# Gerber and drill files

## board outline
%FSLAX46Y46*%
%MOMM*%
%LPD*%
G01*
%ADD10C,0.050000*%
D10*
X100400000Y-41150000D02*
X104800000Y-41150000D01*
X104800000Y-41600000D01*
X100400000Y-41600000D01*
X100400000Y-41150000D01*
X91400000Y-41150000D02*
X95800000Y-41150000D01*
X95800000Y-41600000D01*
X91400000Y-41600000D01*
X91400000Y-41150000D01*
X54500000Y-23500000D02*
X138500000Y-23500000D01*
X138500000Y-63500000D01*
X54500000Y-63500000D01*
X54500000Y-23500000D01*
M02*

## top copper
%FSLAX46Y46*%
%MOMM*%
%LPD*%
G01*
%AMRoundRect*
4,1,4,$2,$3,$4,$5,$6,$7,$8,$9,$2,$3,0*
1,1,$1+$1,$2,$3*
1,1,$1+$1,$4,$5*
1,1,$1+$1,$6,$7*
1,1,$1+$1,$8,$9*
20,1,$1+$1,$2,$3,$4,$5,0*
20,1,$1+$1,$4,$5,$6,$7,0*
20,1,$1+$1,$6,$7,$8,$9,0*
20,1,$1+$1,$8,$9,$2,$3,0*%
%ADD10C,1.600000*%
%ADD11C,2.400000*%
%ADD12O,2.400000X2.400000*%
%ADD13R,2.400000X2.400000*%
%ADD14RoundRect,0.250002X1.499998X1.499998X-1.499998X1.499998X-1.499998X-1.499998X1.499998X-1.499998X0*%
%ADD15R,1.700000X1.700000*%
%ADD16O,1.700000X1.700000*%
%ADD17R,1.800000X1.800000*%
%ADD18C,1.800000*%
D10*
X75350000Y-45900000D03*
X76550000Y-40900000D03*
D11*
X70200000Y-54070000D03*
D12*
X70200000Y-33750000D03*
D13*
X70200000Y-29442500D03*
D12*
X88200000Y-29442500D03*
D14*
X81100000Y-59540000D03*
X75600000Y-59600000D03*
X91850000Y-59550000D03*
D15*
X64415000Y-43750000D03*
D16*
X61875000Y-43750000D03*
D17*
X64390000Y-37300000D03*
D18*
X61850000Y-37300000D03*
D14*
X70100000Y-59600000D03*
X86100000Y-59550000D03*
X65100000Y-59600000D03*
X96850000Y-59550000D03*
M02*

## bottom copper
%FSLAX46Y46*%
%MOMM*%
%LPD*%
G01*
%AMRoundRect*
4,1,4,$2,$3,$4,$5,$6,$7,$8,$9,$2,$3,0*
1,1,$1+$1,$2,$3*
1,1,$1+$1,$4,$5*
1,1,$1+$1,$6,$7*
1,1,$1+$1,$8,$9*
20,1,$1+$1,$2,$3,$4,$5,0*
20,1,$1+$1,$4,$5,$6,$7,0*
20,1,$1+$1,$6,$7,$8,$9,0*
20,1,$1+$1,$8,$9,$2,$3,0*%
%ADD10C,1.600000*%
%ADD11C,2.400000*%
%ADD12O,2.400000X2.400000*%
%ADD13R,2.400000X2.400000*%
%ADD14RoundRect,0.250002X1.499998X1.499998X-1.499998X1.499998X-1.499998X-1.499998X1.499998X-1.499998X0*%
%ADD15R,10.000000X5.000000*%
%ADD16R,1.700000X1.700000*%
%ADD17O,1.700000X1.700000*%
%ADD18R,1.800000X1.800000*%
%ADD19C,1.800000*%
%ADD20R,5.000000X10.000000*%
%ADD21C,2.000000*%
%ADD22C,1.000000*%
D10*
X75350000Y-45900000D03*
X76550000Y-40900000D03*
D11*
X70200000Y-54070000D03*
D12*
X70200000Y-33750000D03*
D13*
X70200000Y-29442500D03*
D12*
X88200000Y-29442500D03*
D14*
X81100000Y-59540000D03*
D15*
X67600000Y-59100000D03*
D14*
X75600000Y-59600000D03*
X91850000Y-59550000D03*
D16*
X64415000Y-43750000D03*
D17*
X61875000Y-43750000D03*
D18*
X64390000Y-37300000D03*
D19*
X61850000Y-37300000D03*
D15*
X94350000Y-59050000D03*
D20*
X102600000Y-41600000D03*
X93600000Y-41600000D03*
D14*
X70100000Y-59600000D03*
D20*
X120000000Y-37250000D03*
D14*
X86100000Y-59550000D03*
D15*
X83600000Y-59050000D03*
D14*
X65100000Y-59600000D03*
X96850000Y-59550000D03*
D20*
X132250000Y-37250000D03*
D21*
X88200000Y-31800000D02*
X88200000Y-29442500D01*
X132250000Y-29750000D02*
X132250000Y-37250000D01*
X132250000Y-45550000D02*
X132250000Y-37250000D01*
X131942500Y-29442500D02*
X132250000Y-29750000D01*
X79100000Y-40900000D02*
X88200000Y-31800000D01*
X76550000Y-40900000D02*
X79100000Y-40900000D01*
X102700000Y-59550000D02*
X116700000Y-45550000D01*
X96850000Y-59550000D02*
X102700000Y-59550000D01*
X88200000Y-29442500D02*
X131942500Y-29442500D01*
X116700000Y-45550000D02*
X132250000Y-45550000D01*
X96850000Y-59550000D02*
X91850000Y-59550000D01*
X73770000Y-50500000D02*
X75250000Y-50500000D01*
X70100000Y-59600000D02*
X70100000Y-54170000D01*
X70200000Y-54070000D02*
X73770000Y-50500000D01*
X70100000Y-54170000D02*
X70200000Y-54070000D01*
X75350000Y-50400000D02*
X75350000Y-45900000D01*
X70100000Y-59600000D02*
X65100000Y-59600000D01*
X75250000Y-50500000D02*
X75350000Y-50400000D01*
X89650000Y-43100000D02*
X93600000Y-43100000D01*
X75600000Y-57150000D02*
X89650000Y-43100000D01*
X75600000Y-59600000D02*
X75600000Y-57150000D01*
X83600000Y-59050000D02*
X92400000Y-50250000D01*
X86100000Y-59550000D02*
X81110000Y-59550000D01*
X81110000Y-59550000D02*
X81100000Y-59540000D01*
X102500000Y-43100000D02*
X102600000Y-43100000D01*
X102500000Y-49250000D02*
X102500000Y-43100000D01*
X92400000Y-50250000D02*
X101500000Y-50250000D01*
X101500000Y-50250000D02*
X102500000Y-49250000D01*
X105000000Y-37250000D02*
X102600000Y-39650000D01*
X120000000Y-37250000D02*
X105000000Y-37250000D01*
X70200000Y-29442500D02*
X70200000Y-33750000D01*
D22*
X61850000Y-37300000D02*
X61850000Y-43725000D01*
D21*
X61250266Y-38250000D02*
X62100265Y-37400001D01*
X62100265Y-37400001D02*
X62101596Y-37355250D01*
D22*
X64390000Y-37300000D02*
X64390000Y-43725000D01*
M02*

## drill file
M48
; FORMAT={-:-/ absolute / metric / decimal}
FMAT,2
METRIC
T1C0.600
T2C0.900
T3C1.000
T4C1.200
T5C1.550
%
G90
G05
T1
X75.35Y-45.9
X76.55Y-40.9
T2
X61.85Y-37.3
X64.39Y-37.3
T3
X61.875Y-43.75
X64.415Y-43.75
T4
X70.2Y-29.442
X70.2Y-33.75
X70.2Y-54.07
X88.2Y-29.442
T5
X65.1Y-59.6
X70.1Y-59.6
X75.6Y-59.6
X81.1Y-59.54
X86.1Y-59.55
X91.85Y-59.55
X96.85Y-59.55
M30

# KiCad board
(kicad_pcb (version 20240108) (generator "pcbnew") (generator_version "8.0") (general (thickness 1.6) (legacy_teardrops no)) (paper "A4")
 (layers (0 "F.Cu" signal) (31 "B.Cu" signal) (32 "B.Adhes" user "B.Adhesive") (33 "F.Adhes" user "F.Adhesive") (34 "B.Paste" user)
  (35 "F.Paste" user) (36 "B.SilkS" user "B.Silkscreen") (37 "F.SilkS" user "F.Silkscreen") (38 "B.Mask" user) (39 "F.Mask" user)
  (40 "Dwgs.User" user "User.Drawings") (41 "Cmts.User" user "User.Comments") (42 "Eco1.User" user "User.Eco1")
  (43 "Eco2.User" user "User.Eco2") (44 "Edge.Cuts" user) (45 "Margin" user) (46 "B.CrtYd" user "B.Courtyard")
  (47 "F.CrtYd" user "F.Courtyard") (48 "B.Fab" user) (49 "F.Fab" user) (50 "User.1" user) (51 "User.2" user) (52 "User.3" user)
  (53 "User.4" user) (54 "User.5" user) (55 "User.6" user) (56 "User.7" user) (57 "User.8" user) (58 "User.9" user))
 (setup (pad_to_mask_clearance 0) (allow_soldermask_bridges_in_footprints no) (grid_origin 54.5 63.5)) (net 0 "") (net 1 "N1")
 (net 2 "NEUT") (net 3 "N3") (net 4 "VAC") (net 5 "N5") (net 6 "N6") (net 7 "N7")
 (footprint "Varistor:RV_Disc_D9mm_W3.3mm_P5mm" (layer "F.Cu") (at 75.35 45.9 90)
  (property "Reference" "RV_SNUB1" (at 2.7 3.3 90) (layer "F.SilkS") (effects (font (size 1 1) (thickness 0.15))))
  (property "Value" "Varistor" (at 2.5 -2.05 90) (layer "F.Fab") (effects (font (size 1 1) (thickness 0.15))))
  (pad "1" thru_hole circle (at 0 0 90) (size 1.6 1.6) (drill 0.6) (layers "*.Cu" "*.Mask") (remove_unused_layers no) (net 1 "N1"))
  (pad "2" thru_hole circle (at 5 1.2 90) (size 1.6 1.6) (drill 0.6) (layers "*.Cu" "*.Mask") (remove_unused_layers no) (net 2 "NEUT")))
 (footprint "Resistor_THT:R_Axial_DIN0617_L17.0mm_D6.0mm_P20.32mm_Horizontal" (layer "F.Cu") (at 70.2 54.07 90)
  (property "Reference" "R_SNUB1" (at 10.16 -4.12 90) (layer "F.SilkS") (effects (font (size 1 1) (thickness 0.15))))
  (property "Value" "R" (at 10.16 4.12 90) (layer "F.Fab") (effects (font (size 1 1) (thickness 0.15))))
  (pad "1" thru_hole circle (at 0 0 90) (size 2.4 2.4) (drill 1.2) (layers "*.Cu" "*.Mask") (remove_unused_layers no) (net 1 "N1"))
  (pad "2" thru_hole oval (at 20.32 0 90) (size 2.4 2.4) (drill 1.2) (layers "*.Cu" "*.Mask") (remove_unused_layers no) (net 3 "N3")))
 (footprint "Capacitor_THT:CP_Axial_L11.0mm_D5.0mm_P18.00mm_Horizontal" (layer "F.Cu") (at 70.2 29.4425)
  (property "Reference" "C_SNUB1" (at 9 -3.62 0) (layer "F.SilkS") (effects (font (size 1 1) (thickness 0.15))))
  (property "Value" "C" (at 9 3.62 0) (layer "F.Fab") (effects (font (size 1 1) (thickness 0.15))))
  (pad "1" thru_hole rect (at 0 0) (size 2.4 2.4) (drill 1.2) (layers "*.Cu" "*.Mask") (remove_unused_layers no) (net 3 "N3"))
  (pad "2" thru_hole oval (at 18 0) (size 2.4 2.4) (drill 1.2) (layers "*.Cu" "*.Mask") (remove_unused_layers no) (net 2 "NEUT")))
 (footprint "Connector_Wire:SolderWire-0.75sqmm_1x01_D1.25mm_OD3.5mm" (layer "B.Cu") (at 81.1 59.54 180)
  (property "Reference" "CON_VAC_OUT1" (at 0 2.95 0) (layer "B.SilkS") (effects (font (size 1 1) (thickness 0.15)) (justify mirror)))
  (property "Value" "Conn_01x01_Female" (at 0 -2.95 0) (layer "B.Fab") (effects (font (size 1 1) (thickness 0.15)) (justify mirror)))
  (pad "1" thru_hole roundrect (at 0 0 180) (size 3.5 3.5) (drill 1.55) (layers "*.Cu" "*.Mask") (remove_unused_layers no)
   (roundrect_rratio 0.071429) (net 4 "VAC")))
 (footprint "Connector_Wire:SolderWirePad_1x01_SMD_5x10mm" (layer "B.Cu") (at 67.6 59.1 90)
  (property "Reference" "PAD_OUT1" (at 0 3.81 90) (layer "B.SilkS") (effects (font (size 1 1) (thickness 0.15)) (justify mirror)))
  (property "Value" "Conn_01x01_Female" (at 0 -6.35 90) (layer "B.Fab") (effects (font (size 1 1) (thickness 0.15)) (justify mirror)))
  (pad "1" smd rect (at 0 0 90) (size 5 10) (layers "B.Cu" "B.Paste" "B.Mask") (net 1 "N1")))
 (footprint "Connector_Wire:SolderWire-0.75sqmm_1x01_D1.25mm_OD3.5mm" (layer "B.Cu") (at 75.6 59.6 180)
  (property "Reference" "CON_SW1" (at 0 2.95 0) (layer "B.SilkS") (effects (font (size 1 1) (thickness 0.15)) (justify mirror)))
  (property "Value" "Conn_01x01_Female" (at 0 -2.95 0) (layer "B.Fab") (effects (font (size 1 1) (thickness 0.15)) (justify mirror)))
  (pad "1" thru_hole roundrect (at 0 0 180) (size 3.5 3.5) (drill 1.55) (layers "*.Cu" "*.Mask") (remove_unused_layers no)
   (roundrect_rratio 0.071429) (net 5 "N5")))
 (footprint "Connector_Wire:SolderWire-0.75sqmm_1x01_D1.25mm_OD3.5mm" (layer "B.Cu") (at 91.85 59.55 180)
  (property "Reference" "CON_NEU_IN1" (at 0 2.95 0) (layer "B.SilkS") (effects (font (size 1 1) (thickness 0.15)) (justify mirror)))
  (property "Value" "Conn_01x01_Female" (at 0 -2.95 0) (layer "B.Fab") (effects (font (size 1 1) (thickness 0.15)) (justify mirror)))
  (pad "1" thru_hole roundrect (at 0 0 180) (size 3.5 3.5) (drill 1.55) (layers "*.Cu" "*.Mask") (remove_unused_layers no)
   (roundrect_rratio 0.071429) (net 2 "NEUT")))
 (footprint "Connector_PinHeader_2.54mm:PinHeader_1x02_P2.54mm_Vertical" (layer "B.Cu") (at 64.415 43.75 90)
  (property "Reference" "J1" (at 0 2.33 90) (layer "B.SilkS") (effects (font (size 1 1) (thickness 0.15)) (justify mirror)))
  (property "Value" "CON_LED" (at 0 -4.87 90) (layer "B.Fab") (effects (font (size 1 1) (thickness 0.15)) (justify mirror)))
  (pad "1" thru_hole rect (at 0 0 90) (size 1.7 1.7) (drill 1) (layers "*.Cu" "*.Mask") (remove_unused_layers no) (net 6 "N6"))
  (pad "2" thru_hole oval (at 0 -2.54 90) (size 1.7 1.7) (drill 1) (layers "*.Cu" "*.Mask") (remove_unused_layers no) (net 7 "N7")))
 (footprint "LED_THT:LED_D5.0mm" (layer "B.Cu") (at 64.39 37.3 180)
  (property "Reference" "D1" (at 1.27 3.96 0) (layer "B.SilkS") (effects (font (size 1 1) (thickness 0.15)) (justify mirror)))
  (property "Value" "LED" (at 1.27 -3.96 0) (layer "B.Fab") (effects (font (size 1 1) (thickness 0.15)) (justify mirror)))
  (pad "1" thru_hole rect (at 0 0 180) (size 1.8 1.8) (drill 0.9) (layers "*.Cu" "*.Mask") (remove_unused_layers no) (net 6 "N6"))
  (pad "2" thru_hole circle (at 2.54 0 180) (size 1.8 1.8) (drill 0.9) (layers "*.Cu" "*.Mask") (remove_unused_layers no) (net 7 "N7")))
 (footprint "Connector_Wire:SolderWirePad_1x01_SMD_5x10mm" (layer "B.Cu") (at 94.35 59.05 90)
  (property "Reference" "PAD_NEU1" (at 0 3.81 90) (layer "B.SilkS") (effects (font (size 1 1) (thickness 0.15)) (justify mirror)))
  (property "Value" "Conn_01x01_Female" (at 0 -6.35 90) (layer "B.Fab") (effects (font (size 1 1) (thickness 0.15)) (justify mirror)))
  (pad "1" smd rect (at 0 0 90) (size 5 10) (layers "B.Cu" "B.Paste" "B.Mask") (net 2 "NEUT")))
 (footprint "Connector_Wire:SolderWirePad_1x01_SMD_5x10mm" (layer "B.Cu") (at 102.6 41.6 180)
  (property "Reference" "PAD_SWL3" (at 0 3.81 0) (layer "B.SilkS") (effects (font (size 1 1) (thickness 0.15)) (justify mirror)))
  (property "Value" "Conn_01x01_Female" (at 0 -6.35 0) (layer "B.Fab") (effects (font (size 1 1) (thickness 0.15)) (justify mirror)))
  (pad "1" smd rect (at 0 0 180) (size 5 10) (layers "B.Cu" "B.Paste" "B.Mask") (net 4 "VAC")))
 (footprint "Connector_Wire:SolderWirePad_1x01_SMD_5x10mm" (layer "B.Cu") (at 93.6 41.6 180)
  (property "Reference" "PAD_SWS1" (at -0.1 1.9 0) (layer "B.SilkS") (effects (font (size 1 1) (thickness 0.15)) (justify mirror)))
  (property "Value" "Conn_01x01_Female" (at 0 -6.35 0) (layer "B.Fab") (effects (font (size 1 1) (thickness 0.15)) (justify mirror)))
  (pad "1" smd rect (at 0 0 180) (size 5 10) (layers "B.Cu" "B.Paste" "B.Mask") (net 5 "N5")))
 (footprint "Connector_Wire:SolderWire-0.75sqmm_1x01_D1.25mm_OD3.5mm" (layer "B.Cu") (at 70.1 59.6 180)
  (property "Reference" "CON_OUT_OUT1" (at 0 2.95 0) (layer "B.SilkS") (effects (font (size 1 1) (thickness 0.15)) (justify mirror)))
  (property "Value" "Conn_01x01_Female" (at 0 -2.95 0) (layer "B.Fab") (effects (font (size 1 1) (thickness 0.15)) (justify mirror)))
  (pad "1" thru_hole roundrect (at 0 0 180) (size 3.5 3.5) (drill 1.55) (layers "*.Cu" "*.Mask") (remove_unused_layers no)
   (roundrect_rratio 0.071429) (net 1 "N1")))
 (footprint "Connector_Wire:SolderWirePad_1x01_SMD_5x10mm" (layer "B.Cu") (at 120 37.25 180)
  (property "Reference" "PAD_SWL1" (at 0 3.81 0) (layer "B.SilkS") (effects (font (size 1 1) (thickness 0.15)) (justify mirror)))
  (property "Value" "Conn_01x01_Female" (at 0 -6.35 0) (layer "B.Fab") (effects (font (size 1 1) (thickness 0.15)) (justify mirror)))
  (pad "1" smd rect (at 0 0 180) (size 5 10) (layers "B.Cu" "B.Paste" "B.Mask") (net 4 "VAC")))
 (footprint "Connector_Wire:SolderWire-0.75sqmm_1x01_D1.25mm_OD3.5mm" (layer "B.Cu") (at 86.1 59.55 180)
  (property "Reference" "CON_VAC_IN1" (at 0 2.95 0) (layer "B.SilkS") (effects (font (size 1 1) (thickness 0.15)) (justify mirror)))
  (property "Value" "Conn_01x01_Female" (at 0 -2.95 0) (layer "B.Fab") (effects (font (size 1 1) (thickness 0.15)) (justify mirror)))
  (pad "1" thru_hole roundrect (at 0 0 180) (size 3.5 3.5) (drill 1.55) (layers "*.Cu" "*.Mask") (remove_unused_layers no)
   (roundrect_rratio 0.071429) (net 4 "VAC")))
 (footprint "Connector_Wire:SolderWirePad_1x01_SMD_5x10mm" (layer "B.Cu") (at 83.6 59.05 90)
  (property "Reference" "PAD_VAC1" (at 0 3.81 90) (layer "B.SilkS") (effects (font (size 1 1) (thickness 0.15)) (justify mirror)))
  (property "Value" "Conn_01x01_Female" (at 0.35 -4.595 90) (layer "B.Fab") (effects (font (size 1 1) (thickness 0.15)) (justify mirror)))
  (pad "1" smd rect (at 0 0 90) (size 5 10) (layers "B.Cu" "B.Paste" "B.Mask") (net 4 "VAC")))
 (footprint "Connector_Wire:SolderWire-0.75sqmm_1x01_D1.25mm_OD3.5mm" (layer "B.Cu") (at 65.1 59.6 180)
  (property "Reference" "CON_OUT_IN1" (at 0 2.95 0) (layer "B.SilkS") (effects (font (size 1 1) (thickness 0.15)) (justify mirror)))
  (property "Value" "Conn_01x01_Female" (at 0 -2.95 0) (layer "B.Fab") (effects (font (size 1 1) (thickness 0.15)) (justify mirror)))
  (pad "1" thru_hole roundrect (at 0 0 180) (size 3.5 3.5) (drill 1.55) (layers "*.Cu" "*.Mask") (remove_unused_layers no)
   (roundrect_rratio 0.071429) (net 1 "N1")))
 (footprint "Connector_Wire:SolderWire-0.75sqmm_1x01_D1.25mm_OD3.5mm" (layer "B.Cu") (at 96.85 59.55 180)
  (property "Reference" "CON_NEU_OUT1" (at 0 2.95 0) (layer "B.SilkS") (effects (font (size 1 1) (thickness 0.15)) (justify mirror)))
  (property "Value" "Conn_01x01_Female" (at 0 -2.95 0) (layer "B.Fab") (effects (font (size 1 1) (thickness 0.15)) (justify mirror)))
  (pad "1" thru_hole roundrect (at 0 0 180) (size 3.5 3.5) (drill 1.55) (layers "*.Cu" "*.Mask") (remove_unused_layers no)
   (roundrect_rratio 0.071429) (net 2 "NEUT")))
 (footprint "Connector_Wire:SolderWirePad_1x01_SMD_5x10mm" (layer "B.Cu") (at 132.25 37.25 180)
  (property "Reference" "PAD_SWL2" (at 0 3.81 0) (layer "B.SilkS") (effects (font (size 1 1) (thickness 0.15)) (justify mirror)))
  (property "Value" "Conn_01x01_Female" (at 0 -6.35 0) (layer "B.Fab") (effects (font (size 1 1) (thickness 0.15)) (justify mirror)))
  (pad "1" smd rect (at 0 0 180) (size 5 10) (layers "B.Cu" "B.Paste" "B.Mask") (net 2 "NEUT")))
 (gr_rect (start 100.4 41.15) (end 104.8 41.6) (stroke (width 0.05) (type default)) (fill none) (layer "Edge.Cuts"))
 (gr_rect (start 91.4 41.15) (end 95.8 41.6) (stroke (width 0.05) (type default)) (fill none) (layer "Edge.Cuts"))
 (gr_rect (start 54.5 23.5) (end 138.5 63.5) (stroke (width 0.05) (type default)) (fill none) (layer "Edge.Cuts"))
 (segment (start 88.2 31.8) (end 88.2 29.4425) (width 2) (layer "B.Cu") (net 2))
 (segment (start 132.25 29.75) (end 132.25 37.25) (width 2) (layer "B.Cu") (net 2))
 (segment (start 132.25 45.55) (end 132.25 37.25) (width 2) (layer "B.Cu") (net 2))
 (segment (start 131.9425 29.4425) (end 132.25 29.75) (width 2) (layer "B.Cu") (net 2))
 (segment (start 79.1 40.9) (end 88.2 31.8) (width 2) (layer "B.Cu") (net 2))
 (segment (start 76.55 40.9) (end 79.1 40.9) (width 2) (layer "B.Cu") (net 2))
 (segment (start 102.7 59.55) (end 116.7 45.55) (width 2) (layer "B.Cu") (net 2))
 (segment (start 96.85 59.55) (end 102.7 59.55) (width 2) (layer "B.Cu") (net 2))
 (segment (start 88.2 29.4425) (end 131.9425 29.4425) (width 2) (layer "B.Cu") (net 2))
 (segment (start 116.7 45.55) (end 132.25 45.55) (width 2) (layer "B.Cu") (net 2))
 (segment (start 96.85 59.55) (end 91.85 59.55) (width 2) (layer "B.Cu") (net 2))
 (segment (start 73.77 50.5) (end 75.25 50.5) (width 2) (layer "B.Cu") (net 1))
 (segment (start 70.1 59.6) (end 70.1 54.17) (width 2) (layer "B.Cu") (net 1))
 (segment (start 70.2 54.07) (end 73.77 50.5) (width 2) (layer "B.Cu") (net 1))
 (segment (start 70.1 54.17) (end 70.2 54.07) (width 2) (layer "B.Cu") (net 1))
 (segment (start 75.35 50.4) (end 75.35 45.9) (width 2) (layer "B.Cu") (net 1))
 (segment (start 70.1 59.6) (end 65.1 59.6) (width 2) (layer "B.Cu") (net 1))
 (segment (start 75.25 50.5) (end 75.35 50.4) (width 2) (layer "B.Cu") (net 1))
 (segment (start 89.65 43.1) (end 93.6 43.1) (width 2) (layer "B.Cu") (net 5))
 (segment (start 75.6 57.15) (end 89.65 43.1) (width 2) (layer "B.Cu") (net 5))
 (segment (start 75.6 59.6) (end 75.6 57.15) (width 2) (layer "B.Cu") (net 5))
 (segment (start 83.6 59.05) (end 92.4 50.25) (width 2) (layer "B.Cu") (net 4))
 (segment (start 86.1 59.55) (end 81.11 59.55) (width 2) (layer "B.Cu") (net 4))
 (segment (start 81.11 59.55) (end 81.1 59.54) (width 2) (layer "B.Cu") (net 4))
 (segment (start 102.5 43.1) (end 102.6 43.1) (width 2) (layer "B.Cu") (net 4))
 (segment (start 102.5 49.25) (end 102.5 43.1) (width 2) (layer "B.Cu") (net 4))
 (segment (start 92.4 50.25) (end 101.5 50.25) (width 2) (layer "B.Cu") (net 4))
 (segment (start 101.5 50.25) (end 102.5 49.25) (width 2) (layer "B.Cu") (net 4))
 (segment (start 105 37.25) (end 102.6 39.65) (width 2) (layer "B.Cu") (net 4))
 (segment (start 120 37.25) (end 105 37.25) (width 2) (layer "B.Cu") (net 4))
 (segment (start 70.2 29.4425) (end 70.2 33.75) (width 2) (layer "B.Cu") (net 3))
 (segment (start 61.85 37.3) (end 61.85 43.725) (width 1) (layer "B.Cu") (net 7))
 (segment (start 61.250266 38.25) (end 62.100265 37.400001) (width 2) (layer "B.Cu") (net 7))
 (segment (start 62.100265 37.400001) (end 62.101596 37.35525) (width 2) (layer "B.Cu") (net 7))
 (segment (start 64.39 37.3) (end 64.39 43.725) (width 1) (layer "B.Cu") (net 6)))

